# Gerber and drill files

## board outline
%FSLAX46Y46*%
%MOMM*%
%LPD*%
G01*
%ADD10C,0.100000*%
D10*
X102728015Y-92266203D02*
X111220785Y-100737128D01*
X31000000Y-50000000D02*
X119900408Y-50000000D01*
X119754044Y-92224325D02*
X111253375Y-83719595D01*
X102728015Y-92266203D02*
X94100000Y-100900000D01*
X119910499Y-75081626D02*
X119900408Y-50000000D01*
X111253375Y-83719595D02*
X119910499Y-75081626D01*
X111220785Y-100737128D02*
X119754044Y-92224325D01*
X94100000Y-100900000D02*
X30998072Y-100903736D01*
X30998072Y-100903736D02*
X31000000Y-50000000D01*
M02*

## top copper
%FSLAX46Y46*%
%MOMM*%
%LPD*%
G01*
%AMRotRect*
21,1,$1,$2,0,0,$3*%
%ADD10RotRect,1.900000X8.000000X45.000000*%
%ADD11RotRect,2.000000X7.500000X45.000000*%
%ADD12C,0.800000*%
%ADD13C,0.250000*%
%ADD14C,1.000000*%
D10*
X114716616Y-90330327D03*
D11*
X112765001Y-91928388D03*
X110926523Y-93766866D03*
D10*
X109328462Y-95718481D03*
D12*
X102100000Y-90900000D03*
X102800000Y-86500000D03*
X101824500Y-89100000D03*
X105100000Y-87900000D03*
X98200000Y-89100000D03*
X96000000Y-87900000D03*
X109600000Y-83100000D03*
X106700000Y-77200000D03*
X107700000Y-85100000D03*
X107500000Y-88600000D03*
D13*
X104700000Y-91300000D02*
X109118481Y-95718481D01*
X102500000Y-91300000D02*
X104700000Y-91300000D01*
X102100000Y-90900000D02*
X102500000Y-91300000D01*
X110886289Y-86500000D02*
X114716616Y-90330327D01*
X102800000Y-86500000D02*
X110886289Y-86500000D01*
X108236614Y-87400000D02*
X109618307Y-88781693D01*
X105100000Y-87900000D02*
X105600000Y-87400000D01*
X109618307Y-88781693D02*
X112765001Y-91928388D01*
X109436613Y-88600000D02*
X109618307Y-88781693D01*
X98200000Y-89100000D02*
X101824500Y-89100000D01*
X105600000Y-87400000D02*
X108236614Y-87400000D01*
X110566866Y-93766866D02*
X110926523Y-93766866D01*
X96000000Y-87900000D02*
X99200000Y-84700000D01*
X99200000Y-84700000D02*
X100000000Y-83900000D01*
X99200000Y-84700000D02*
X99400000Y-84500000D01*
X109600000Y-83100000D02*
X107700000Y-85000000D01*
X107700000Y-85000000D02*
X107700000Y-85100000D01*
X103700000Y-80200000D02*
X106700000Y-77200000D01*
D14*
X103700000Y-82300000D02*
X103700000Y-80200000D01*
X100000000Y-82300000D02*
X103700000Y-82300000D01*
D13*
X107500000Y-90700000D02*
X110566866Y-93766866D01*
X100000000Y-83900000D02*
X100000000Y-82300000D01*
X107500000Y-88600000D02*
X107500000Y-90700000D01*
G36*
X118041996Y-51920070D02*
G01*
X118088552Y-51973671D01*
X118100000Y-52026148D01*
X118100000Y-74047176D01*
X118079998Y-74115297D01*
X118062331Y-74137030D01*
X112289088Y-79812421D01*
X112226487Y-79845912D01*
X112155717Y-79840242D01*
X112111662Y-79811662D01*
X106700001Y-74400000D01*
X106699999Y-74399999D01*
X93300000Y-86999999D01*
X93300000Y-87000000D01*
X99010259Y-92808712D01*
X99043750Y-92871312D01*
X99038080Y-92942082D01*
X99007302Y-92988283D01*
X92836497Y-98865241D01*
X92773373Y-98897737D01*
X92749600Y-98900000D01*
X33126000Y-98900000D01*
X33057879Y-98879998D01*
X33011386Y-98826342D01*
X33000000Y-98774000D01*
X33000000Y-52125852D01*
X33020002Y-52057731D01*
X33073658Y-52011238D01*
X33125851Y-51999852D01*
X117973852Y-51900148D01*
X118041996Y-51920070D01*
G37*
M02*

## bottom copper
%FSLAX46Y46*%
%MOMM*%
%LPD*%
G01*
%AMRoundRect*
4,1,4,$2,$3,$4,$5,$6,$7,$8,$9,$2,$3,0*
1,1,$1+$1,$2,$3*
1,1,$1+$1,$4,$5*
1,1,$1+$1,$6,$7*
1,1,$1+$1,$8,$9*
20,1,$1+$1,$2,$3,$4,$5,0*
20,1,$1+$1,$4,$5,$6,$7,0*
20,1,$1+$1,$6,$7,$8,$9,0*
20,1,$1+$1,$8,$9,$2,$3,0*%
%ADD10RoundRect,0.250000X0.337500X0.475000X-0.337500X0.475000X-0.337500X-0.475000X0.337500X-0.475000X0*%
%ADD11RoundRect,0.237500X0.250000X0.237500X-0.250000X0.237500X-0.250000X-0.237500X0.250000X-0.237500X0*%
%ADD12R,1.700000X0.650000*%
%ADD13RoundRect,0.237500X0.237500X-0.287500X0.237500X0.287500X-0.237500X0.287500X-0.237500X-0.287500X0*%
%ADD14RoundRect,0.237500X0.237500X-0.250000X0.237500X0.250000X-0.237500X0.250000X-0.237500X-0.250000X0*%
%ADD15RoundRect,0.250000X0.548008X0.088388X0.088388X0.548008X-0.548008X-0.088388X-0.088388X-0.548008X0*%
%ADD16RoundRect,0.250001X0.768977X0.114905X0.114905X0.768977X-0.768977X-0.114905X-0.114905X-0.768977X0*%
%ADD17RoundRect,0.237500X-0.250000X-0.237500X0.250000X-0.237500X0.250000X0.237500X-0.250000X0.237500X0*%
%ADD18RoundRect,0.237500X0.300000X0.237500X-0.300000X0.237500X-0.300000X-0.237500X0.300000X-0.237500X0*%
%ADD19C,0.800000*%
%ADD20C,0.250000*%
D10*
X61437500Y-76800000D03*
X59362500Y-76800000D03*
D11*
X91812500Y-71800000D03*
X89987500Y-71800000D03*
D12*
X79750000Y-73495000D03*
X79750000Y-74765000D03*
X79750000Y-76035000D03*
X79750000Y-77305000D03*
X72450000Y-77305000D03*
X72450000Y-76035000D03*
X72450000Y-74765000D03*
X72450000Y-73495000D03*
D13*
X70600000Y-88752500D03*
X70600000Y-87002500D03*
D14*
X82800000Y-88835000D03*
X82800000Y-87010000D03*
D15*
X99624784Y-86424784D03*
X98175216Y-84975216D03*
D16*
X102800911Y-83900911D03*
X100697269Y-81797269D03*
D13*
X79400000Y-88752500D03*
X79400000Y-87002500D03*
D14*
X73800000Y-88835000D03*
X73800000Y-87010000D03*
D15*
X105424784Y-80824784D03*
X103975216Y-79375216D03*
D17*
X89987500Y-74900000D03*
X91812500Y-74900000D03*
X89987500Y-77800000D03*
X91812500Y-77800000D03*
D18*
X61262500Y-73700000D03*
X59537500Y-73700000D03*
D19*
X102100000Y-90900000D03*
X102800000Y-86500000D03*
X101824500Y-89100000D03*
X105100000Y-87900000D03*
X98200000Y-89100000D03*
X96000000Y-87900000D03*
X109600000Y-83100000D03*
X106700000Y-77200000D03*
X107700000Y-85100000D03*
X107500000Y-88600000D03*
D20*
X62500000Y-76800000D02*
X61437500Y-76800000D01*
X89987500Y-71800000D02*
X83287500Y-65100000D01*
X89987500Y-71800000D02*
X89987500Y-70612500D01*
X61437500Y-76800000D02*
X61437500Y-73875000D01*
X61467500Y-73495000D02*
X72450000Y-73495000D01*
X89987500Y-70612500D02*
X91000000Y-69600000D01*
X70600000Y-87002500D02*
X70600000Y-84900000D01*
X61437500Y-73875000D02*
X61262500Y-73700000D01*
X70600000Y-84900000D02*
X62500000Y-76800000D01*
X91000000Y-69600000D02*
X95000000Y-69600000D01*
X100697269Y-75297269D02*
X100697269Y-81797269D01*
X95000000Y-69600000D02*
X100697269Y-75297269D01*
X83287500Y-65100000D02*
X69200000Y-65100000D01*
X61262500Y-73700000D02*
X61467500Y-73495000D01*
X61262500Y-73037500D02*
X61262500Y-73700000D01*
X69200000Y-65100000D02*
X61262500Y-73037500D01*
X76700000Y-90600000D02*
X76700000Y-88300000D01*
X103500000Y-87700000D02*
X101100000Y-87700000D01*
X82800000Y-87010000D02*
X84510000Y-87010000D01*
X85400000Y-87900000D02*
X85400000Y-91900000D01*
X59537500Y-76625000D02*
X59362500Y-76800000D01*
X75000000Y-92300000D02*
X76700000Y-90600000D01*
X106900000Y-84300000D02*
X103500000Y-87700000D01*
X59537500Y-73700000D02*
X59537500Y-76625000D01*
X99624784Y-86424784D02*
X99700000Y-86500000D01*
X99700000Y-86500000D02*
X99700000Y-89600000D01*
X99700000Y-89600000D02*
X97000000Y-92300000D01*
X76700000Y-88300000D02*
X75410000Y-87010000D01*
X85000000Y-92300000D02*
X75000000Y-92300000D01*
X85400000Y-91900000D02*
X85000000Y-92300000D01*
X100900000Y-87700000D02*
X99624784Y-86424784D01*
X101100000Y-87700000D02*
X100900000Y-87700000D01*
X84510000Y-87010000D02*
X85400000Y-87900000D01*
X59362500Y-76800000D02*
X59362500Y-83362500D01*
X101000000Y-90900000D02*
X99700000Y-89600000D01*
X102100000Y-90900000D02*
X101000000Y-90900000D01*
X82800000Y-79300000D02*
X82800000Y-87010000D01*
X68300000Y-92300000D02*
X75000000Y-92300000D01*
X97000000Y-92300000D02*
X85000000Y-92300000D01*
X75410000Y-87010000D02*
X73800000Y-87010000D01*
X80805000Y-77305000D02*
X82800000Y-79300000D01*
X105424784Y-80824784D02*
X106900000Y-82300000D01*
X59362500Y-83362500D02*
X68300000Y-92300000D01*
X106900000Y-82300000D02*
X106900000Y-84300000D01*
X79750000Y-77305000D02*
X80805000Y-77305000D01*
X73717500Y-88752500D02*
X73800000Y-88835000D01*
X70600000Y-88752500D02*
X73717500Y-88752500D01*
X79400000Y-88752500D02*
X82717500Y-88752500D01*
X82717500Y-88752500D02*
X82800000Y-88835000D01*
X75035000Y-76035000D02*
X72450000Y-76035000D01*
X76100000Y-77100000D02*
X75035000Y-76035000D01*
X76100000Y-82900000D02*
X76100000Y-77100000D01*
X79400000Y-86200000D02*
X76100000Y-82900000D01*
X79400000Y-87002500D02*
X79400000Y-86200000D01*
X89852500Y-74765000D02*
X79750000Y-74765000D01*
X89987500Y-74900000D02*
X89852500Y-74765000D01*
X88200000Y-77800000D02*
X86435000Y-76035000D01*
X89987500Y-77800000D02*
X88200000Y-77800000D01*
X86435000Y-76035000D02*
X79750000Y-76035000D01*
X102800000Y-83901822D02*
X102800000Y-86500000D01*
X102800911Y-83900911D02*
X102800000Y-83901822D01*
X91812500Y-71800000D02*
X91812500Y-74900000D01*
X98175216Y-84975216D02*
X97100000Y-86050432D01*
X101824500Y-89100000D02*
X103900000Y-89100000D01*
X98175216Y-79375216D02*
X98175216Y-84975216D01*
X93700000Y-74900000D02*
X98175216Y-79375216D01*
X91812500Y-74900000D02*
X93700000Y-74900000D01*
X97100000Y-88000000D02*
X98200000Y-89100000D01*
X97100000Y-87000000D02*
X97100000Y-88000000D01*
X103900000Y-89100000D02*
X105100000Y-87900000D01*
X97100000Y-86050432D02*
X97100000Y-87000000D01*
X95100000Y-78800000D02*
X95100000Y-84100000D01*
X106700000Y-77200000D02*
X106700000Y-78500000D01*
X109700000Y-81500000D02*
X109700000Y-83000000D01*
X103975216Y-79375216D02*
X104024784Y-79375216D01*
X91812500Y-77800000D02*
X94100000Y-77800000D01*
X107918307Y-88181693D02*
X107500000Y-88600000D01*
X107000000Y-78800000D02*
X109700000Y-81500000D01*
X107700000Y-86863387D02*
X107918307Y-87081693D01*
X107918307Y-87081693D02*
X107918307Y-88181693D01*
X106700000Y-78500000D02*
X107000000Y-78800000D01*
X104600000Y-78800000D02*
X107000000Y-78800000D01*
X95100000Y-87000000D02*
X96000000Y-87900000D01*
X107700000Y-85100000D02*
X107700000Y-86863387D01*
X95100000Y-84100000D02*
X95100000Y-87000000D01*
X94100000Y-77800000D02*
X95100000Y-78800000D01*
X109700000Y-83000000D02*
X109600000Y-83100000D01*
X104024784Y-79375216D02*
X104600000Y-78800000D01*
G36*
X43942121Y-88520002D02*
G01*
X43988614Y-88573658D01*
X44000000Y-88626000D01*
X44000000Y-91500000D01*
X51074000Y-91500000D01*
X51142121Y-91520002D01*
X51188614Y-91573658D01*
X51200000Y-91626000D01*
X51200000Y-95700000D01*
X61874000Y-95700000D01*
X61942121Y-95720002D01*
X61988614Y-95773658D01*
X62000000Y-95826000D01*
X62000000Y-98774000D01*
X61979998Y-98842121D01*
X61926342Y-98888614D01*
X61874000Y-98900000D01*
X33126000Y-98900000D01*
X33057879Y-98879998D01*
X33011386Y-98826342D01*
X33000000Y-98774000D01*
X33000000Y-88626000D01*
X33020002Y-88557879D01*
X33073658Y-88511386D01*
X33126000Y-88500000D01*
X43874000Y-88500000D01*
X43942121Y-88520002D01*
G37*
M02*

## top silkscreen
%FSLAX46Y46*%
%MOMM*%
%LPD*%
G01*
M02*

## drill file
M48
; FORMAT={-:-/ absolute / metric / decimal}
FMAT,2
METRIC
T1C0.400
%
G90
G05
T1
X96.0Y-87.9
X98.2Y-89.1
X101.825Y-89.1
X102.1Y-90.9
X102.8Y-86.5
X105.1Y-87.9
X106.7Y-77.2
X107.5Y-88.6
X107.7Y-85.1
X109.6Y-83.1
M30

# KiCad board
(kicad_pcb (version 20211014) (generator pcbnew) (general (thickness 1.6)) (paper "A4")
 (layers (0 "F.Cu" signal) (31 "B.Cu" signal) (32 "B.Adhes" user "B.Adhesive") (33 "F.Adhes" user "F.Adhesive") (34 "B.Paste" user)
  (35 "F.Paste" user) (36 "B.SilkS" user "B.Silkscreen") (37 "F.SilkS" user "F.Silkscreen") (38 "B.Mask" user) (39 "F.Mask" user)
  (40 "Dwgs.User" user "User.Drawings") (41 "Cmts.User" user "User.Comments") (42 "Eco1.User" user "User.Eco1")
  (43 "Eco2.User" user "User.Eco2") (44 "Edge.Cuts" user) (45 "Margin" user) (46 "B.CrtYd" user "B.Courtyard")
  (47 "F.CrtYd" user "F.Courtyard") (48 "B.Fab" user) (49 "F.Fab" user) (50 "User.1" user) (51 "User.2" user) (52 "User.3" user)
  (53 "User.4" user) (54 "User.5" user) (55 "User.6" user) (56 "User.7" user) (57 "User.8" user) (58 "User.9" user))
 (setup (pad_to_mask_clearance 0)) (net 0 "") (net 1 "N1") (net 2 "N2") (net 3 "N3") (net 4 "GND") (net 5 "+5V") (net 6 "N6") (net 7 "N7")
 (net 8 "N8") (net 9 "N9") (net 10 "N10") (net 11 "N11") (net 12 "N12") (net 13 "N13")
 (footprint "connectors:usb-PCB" (layer "F.Cu") (at 115.487362 96.489227 45)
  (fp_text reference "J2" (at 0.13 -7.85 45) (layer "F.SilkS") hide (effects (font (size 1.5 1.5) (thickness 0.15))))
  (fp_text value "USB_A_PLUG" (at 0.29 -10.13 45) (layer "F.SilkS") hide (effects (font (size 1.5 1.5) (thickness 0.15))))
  (pad "1" connect rect (at 3.81 -4.9 45) (size 1.9 8) (layers "F.Cu" "F.Mask") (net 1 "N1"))
  (pad "2" connect rect (at 1.3 -5.15 45) (size 2 7.5) (layers "F.Cu" "F.Mask") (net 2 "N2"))
  (pad "3" connect rect (at -1.3 -5.15 45) (size 2 7.5) (layers "F.Cu" "F.Mask") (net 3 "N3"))
  (pad "4" connect rect (at -3.81 -4.9 45) (size 1.9 8) (layers "F.Cu" "F.Mask") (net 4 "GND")))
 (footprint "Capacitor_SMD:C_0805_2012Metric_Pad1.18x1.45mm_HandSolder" (layer "B.Cu") (at 60.4 76.8 180)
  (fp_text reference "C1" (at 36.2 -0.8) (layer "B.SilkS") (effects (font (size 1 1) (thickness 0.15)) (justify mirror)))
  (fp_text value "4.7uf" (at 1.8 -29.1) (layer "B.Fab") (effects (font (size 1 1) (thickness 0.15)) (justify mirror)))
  (pad "1" smd roundrect (at -1.0375 0 180) (size 1.175 1.45) (layers "B.Cu" "B.Paste" "B.Mask") (roundrect_rratio 0.2127659574)
   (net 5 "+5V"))
  (pad "2" smd roundrect (at 1.0375 0 180) (size 1.175 1.45) (layers "B.Cu" "B.Paste" "B.Mask") (roundrect_rratio 0.2127659574)
   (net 4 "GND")))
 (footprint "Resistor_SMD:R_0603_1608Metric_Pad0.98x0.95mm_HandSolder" (layer "B.Cu") (at 90.9 71.8 180)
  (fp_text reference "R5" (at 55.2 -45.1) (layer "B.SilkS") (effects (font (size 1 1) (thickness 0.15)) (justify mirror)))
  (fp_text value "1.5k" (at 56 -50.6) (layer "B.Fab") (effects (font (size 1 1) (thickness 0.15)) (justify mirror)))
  (pad "1" smd roundrect (at -0.9125 0 180) (size 0.975 0.95) (layers "B.Cu" "B.Paste" "B.Mask") (roundrect_rratio 0.25) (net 2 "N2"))
  (pad "2" smd roundrect (at 0.9125 0 180) (size 0.975 0.95) (layers "B.Cu" "B.Paste" "B.Mask") (roundrect_rratio 0.25) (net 5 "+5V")))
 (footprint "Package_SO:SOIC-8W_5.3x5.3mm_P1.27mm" (layer "B.Cu") (at 76.1 75.4 180)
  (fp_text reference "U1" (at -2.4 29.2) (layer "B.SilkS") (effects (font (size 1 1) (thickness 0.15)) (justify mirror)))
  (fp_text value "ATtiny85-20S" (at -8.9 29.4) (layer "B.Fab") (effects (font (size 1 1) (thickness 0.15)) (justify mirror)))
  (pad "1" smd rect (at -3.65 1.905 180) (size 1.7 0.65) (layers "B.Cu" "B.Paste" "B.Mask") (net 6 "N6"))
  (pad "2" smd rect (at -3.65 0.635 180) (size 1.7 0.65) (layers "B.Cu" "B.Paste" "B.Mask") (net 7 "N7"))
  (pad "3" smd rect (at -3.65 -0.635 180) (size 1.7 0.65) (layers "B.Cu" "B.Paste" "B.Mask") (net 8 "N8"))
  (pad "4" smd rect (at -3.65 -1.905 180) (size 1.7 0.65) (layers "B.Cu" "B.Paste" "B.Mask") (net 4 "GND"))
  (pad "5" smd rect (at 3.65 -1.905 180) (size 1.7 0.65) (layers "B.Cu" "B.Paste" "B.Mask") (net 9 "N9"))
  (pad "6" smd rect (at 3.65 -0.635 180) (size 1.7 0.65) (layers "B.Cu" "B.Paste" "B.Mask") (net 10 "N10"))
  (pad "7" smd rect (at 3.65 0.635 180) (size 1.7 0.65) (layers "B.Cu" "B.Paste" "B.Mask") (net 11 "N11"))
  (pad "8" smd rect (at 3.65 1.905 180) (size 1.7 0.65) (layers "B.Cu" "B.Paste" "B.Mask") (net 5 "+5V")))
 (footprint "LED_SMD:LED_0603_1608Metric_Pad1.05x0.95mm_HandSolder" (layer "B.Cu") (at 70.6 87.8775 90)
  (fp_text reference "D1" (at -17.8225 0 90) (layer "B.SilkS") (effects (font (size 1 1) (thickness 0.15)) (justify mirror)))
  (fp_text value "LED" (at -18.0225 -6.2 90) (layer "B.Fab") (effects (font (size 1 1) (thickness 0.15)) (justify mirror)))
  (pad "1" smd roundrect (at -0.875 0 90) (size 1.05 0.95) (layers "B.Cu" "B.Paste" "B.Mask") (roundrect_rratio 0.25) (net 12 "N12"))
  (pad "2" smd roundrect (at 0.875 0 90) (size 1.05 0.95) (layers "B.Cu" "B.Paste" "B.Mask") (roundrect_rratio 0.25) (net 5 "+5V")))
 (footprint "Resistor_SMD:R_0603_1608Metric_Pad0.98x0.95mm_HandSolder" (layer "B.Cu") (at 82.8 87.9225 90)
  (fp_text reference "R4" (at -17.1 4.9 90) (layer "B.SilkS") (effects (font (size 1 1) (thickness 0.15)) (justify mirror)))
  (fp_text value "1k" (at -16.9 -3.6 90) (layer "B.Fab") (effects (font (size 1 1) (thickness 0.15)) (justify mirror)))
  (pad "1" smd roundrect (at -0.9125 0 90) (size 0.975 0.95) (layers "B.Cu" "B.Paste" "B.Mask") (roundrect_rratio 0.25) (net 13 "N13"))
  (pad "2" smd roundrect (at 0.9125 0 90) (size 0.975 0.95) (layers "B.Cu" "B.Paste" "B.Mask") (roundrect_rratio 0.25) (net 4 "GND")))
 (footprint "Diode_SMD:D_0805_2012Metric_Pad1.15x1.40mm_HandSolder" (layer "B.Cu") (at 98.9 85.7 135)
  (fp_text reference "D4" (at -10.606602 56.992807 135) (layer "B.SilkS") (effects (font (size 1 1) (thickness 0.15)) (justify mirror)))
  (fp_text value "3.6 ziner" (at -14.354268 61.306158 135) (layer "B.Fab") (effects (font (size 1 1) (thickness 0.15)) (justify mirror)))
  (pad "1" smd roundrect (at -1.025 0 135) (size 1.15 1.4) (layers "B.Cu" "B.Paste" "B.Mask") (roundrect_rratio 0.2173913043) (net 4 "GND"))
  (pad "2" smd roundrect (at 1.025 0 135) (size 1.15 1.4) (layers "B.Cu" "B.Paste" "B.Mask") (roundrect_rratio 0.2173913043) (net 2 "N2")))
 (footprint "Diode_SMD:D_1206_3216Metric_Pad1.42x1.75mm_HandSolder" (layer "B.Cu") (at 101.74909 82.84909 135)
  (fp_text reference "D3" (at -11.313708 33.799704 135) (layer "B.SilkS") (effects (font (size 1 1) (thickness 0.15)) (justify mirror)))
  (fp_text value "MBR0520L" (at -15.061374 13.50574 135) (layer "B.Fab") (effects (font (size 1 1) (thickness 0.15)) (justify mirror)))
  (pad "1" smd roundrect (at -1.4875 0 135) (size 1.425 1.75) (layers "B.Cu" "B.Paste" "B.Mask") (roundrect_rratio 0.1754392982)
   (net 1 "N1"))
  (pad "2" smd roundrect (at 1.4875 0 135) (size 1.425 1.75) (layers "B.Cu" "B.Paste" "B.Mask") (roundrect_rratio 0.1754392982)
   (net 5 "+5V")))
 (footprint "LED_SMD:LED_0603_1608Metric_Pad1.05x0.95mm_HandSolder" (layer "B.Cu") (at 79.4 87.8775 90)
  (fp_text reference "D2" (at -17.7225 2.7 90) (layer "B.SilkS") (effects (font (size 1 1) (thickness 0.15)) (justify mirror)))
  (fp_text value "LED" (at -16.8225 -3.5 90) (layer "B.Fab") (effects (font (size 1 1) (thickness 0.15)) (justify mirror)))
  (pad "1" smd roundrect (at -0.875 0 90) (size 1.05 0.95) (layers "B.Cu" "B.Paste" "B.Mask") (roundrect_rratio 0.25) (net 13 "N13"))
  (pad "2" smd roundrect (at 0.875 0 90) (size 1.05 0.95) (layers "B.Cu" "B.Paste" "B.Mask") (roundrect_rratio 0.25) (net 10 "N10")))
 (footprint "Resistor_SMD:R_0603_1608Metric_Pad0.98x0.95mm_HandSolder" (layer "B.Cu") (at 73.8 87.9225 90)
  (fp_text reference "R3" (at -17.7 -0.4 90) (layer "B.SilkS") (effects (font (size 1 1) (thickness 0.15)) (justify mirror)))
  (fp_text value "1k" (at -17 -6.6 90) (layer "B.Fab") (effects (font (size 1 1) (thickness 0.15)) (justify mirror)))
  (pad "1" smd roundrect (at -0.9125 0 90) (size 0.975 0.95) (layers "B.Cu" "B.Paste" "B.Mask") (roundrect_rratio 0.25) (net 12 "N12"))
  (pad "2" smd roundrect (at 0.9125 0 90) (size 0.975 0.95) (layers "B.Cu" "B.Paste" "B.Mask") (roundrect_rratio 0.25) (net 4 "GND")))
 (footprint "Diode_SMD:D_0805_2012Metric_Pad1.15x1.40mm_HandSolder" (layer "B.Cu") (at 104.7 80.1 135)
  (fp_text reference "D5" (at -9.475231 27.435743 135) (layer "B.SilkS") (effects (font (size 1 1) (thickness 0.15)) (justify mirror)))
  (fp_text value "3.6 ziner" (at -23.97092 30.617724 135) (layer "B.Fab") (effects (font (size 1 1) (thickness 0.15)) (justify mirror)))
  (pad "1" smd roundrect (at -1.025 0 135) (size 1.15 1.4) (layers "B.Cu" "B.Paste" "B.Mask") (roundrect_rratio 0.2173913043) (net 4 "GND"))
  (pad "2" smd roundrect (at 1.025 0 135) (size 1.15 1.4) (layers "B.Cu" "B.Paste" "B.Mask") (roundrect_rratio 0.2173913043) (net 3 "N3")))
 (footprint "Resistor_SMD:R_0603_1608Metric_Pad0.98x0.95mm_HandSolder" (layer "B.Cu") (at 90.9 74.9)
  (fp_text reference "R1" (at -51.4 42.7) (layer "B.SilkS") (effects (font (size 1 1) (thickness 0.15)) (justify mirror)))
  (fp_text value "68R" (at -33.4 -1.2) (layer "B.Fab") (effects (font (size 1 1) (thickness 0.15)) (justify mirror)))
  (pad "1" smd roundrect (at -0.9125 0) (size 0.975 0.95) (layers "B.Cu" "B.Paste" "B.Mask") (roundrect_rratio 0.25) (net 7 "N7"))
  (pad "2" smd roundrect (at 0.9125 0) (size 0.975 0.95) (layers "B.Cu" "B.Paste" "B.Mask") (roundrect_rratio 0.25) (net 2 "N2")))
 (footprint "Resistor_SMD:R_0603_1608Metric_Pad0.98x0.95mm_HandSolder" (layer "B.Cu") (at 90.9 77.8)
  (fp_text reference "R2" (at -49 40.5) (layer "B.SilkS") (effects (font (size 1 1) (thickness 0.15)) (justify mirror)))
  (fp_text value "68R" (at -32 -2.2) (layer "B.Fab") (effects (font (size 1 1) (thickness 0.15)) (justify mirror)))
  (pad "1" smd roundrect (at -0.9125 0) (size 0.975 0.95) (layers "B.Cu" "B.Paste" "B.Mask") (roundrect_rratio 0.25) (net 8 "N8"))
  (pad "2" smd roundrect (at 0.9125 0) (size 0.975 0.95) (layers "B.Cu" "B.Paste" "B.Mask") (roundrect_rratio 0.25) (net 3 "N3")))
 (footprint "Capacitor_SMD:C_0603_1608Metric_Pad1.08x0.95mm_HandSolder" (layer "B.Cu") (at 60.4 73.7 180)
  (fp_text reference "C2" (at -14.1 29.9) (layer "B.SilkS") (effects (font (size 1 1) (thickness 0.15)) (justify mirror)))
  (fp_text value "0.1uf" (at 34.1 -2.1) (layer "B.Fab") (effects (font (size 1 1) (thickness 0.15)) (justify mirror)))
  (pad "1" smd roundrect (at -0.8625 0 180) (size 1.075 0.95) (layers "B.Cu" "B.Paste" "B.Mask") (roundrect_rratio 0.25) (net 5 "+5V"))
  (pad "2" smd roundrect (at 0.8625 0 180) (size 1.075 0.95) (layers "B.Cu" "B.Paste" "B.Mask") (roundrect_rratio 0.25) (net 4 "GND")))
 (gr_line (start 102.728015 92.266203) (end 111.220785 100.737128) (layer "Edge.Cuts") (width 0.1))
 (gr_line (start 31 50) (end 119.900408 50) (layer "Edge.Cuts") (width 0.1))
 (gr_line (start 119.754044 92.224325) (end 111.253375 83.719595) (layer "Edge.Cuts") (width 0.1))
 (gr_line (start 102.728015 92.266203) (end 94.1 100.9) (layer "Edge.Cuts") (width 0.1))
 (gr_line (start 119.910499 75.081626) (end 119.900408 50) (layer "Edge.Cuts") (width 0.1))
 (gr_line (start 111.253375 83.719595) (end 119.910499 75.081626) (layer "Edge.Cuts") (width 0.1))
 (gr_line (start 111.220785 100.737128) (end 119.754044 92.224325) (layer "Edge.Cuts") (width 0.1))
 (gr_line (start 94.1 100.9) (end 30.998072 100.903736) (layer "Edge.Cuts") (width 0.1))
 (gr_line (start 30.998072 100.903736) (end 31 50) (layer "Edge.Cuts") (width 0.1))
 (segment (start 62.5 76.8) (end 61.4375 76.8) (width 0.25) (layer "B.Cu") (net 5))
 (segment (start 89.9875 71.8) (end 83.2875 65.1) (width 0.25) (layer "B.Cu") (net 5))
 (segment (start 89.9875 71.8) (end 89.9875 70.6125) (width 0.25) (layer "B.Cu") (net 5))
 (segment (start 61.4375 76.8) (end 61.4375 73.875) (width 0.25) (layer "B.Cu") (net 5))
 (segment (start 61.4675 73.495) (end 72.45 73.495) (width 0.25) (layer "B.Cu") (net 5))
 (segment (start 89.9875 70.6125) (end 91 69.6) (width 0.25) (layer "B.Cu") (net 5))
 (segment (start 70.6 87.0025) (end 70.6 84.9) (width 0.25) (layer "B.Cu") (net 5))
 (segment (start 61.4375 73.875) (end 61.2625 73.7) (width 0.25) (layer "B.Cu") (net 5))
 (segment (start 70.6 84.9) (end 62.5 76.8) (width 0.25) (layer "B.Cu") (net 5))
 (segment (start 91 69.6) (end 95 69.6) (width 0.25) (layer "B.Cu") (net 5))
 (segment (start 100.697269 75.297269) (end 100.697269 81.797269) (width 0.25) (layer "B.Cu") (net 5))
 (segment (start 95 69.6) (end 100.697269 75.297269) (width 0.25) (layer "B.Cu") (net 5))
 (segment (start 83.2875 65.1) (end 69.2 65.1) (width 0.25) (layer "B.Cu") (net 5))
 (segment (start 61.2625 73.7) (end 61.4675 73.495) (width 0.25) (layer "B.Cu") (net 5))
 (segment (start 61.2625 73.0375) (end 61.2625 73.7) (width 0.25) (layer "B.Cu") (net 5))
 (segment (start 69.2 65.1) (end 61.2625 73.0375) (width 0.25) (layer "B.Cu") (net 5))
 (segment (start 104.7 91.3) (end 109.118481 95.718481) (width 0.25) (layer "F.Cu") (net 4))
 (segment (start 102.5 91.3) (end 104.7 91.3) (width 0.25) (layer "F.Cu") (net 4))
 (segment (start 102.1 90.9) (end 102.5 91.3) (width 0.25) (layer "F.Cu") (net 4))
 (via (at 102.1 90.9) (size 0.8) (drill 0.4) (layers "F.Cu" "B.Cu") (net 4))
 (segment (start 76.7 90.6) (end 76.7 88.3) (width 0.25) (layer "B.Cu") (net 4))
 (segment (start 103.5 87.7) (end 101.1 87.7) (width 0.25) (layer "B.Cu") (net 4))
 (segment (start 82.8 87.01) (end 84.51 87.01) (width 0.25) (layer "B.Cu") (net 4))
 (segment (start 85.4 87.9) (end 85.4 91.9) (width 0.25) (layer "B.Cu") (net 4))
 (segment (start 59.5375 76.625) (end 59.3625 76.8) (width 0.25) (layer "B.Cu") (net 4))
 (segment (start 75 92.3) (end 76.7 90.6) (width 0.25) (layer "B.Cu") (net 4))
 (segment (start 106.9 84.3) (end 103.5 87.7) (width 0.25) (layer "B.Cu") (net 4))
 (segment (start 59.5375 73.7) (end 59.5375 76.625) (width 0.25) (layer "B.Cu") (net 4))
 (segment (start 99.624784 86.424784) (end 99.7 86.5) (width 0.25) (layer "B.Cu") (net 4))
 (segment (start 99.7 86.5) (end 99.7 89.6) (width 0.25) (layer "B.Cu") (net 4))
 (segment (start 99.7 89.6) (end 97 92.3) (width 0.25) (layer "B.Cu") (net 4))
 (segment (start 76.7 88.3) (end 75.41 87.01) (width 0.25) (layer "B.Cu") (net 4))
 (segment (start 85 92.3) (end 75 92.3) (width 0.25) (layer "B.Cu") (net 4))
 (segment (start 85.4 91.9) (end 85 92.3) (width 0.25) (layer "B.Cu") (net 4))
 (segment (start 100.9 87.7) (end 99.624784 86.424784) (width 0.25) (layer "B.Cu") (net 4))
 (segment (start 101.1 87.7) (end 100.9 87.7) (width 0.25) (layer "B.Cu") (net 4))
 (segment (start 84.51 87.01) (end 85.4 87.9) (width 0.25) (layer "B.Cu") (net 4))
 (segment (start 59.3625 76.8) (end 59.3625 83.3625) (width 0.25) (layer "B.Cu") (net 4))
 (segment (start 101 90.9) (end 99.7 89.6) (width 0.25) (layer "B.Cu") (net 4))
 (segment (start 102.1 90.9) (end 101 90.9) (width 0.25) (layer "B.Cu") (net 4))
 (segment (start 82.8 79.3) (end 82.8 87.01) (width 0.25) (layer "B.Cu") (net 4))
 (segment (start 68.3 92.3) (end 75 92.3) (width 0.25) (layer "B.Cu") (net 4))
 (segment (start 97 92.3) (end 85 92.3) (width 0.25) (layer "B.Cu") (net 4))
 (segment (start 75.41 87.01) (end 73.8 87.01) (width 0.25) (layer "B.Cu") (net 4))
 (segment (start 80.805 77.305) (end 82.8 79.3) (width 0.25) (layer "B.Cu") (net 4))
 (segment (start 105.424784 80.824784) (end 106.9 82.3) (width 0.25) (layer "B.Cu") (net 4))
 (segment (start 59.3625 83.3625) (end 68.3 92.3) (width 0.25) (layer "B.Cu") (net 4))
 (segment (start 106.9 82.3) (end 106.9 84.3) (width 0.25) (layer "B.Cu") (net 4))
 (segment (start 79.75 77.305) (end 80.805 77.305) (width 0.25) (layer "B.Cu") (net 4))
 (segment (start 73.7175 88.7525) (end 73.8 88.835) (width 0.25) (layer "B.Cu") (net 12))
 (segment (start 70.6 88.7525) (end 73.7175 88.7525) (width 0.25) (layer "B.Cu") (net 12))
 (segment (start 79.4 88.7525) (end 82.7175 88.7525) (width 0.25) (layer "B.Cu") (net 13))
 (segment (start 82.7175 88.7525) (end 82.8 88.835) (width 0.25) (layer "B.Cu") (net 13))
 (segment (start 75.035 76.035) (end 72.45 76.035) (width 0.25) (layer "B.Cu") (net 10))
 (segment (start 76.1 77.1) (end 75.035 76.035) (width 0.25) (layer "B.Cu") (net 10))
 (segment (start 76.1 82.9) (end 76.1 77.1) (width 0.25) (layer "B.Cu") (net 10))
 (segment (start 79.4 86.2) (end 76.1 82.9) (width 0.25) (layer "B.Cu") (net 10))
 (segment (start 79.4 87.0025) (end 79.4 86.2) (width 0.25) (layer "B.Cu") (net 10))
 (segment (start 89.8525 74.765) (end 79.75 74.765) (width 0.25) (layer "B.Cu") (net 7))
 (segment (start 89.9875 74.9) (end 89.8525 74.765) (width 0.25) (layer "B.Cu") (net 7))
 (segment (start 88.2 77.8) (end 86.435 76.035) (width 0.25) (layer "B.Cu") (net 8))
 (segment (start 89.9875 77.8) (end 88.2 77.8) (width 0.25) (layer "B.Cu") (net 8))
 (segment (start 86.435 76.035) (end 79.75 76.035) (width 0.25) (layer "B.Cu") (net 8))
 (segment (start 110.886289 86.5) (end 114.716616 90.330327) (width 0.25) (layer "F.Cu") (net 1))
 (segment (start 102.8 86.5) (end 110.886289 86.5) (width 0.25) (layer "F.Cu") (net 1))
 (via (at 102.8 86.5) (size 0.8) (drill 0.4) (layers "F.Cu" "B.Cu") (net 1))
 (segment (start 102.8 83.901822) (end 102.8 86.5) (width 0.25) (layer "B.Cu") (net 1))
 (segment (start 102.800911 83.900911) (end 102.8 83.901822) (width 0.25) (layer "B.Cu") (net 1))
 (segment (start 108.236614 87.4) (end 109.618307 88.781693) (width 0.25) (layer "F.Cu") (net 2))
 (segment (start 105.1 87.9) (end 105.6 87.4) (width 0.25) (layer "F.Cu") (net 2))
 (segment (start 109.618307 88.781693) (end 112.765001 91.928388) (width 0.25) (layer "F.Cu") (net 2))
 (segment (start 109.436613 88.6) (end 109.618307 88.781693) (width 0.25) (layer "F.Cu") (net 2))
 (segment (start 98.2 89.1) (end 101.8245 89.1) (width 0.25) (layer "F.Cu") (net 2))
 (segment (start 105.6 87.4) (end 108.236614 87.4) (width 0.25) (layer "F.Cu") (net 2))
 (via (at 101.8245 89.1) (size 0.8) (drill 0.4) (layers "F.Cu" "B.Cu") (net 2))
 (via (at 105.1 87.9) (size 0.8) (drill 0.4) (layers "F.Cu" "B.Cu") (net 2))
 (via (at 98.2 89.1) (size 0.8) (drill 0.4) (layers "F.Cu" "B.Cu") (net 2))
 (segment (start 91.8125 71.8) (end 91.8125 74.9) (width 0.25) (layer "B.Cu") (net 2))
 (segment (start 98.175216 84.975216) (end 97.1 86.050432) (width 0.25) (layer "B.Cu") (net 2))
 (segment (start 101.8245 89.1) (end 103.9 89.1) (width 0.25) (layer "B.Cu") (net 2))
 (segment (start 98.175216 79.375216) (end 98.175216 84.975216) (width 0.25) (layer "B.Cu") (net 2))
 (segment (start 93.7 74.9) (end 98.175216 79.375216) (width 0.25) (layer "B.Cu") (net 2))
 (segment (start 91.8125 74.9) (end 93.7 74.9) (width 0.25) (layer "B.Cu") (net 2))
 (segment (start 97.1 88) (end 98.2 89.1) (width 0.25) (layer "B.Cu") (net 2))
 (segment (start 97.1 87) (end 97.1 88) (width 0.25) (layer "B.Cu") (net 2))
 (segment (start 103.9 89.1) (end 105.1 87.9) (width 0.25) (layer "B.Cu") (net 2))
 (segment (start 97.1 86.050432) (end 97.1 87) (width 0.25) (layer "B.Cu") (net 2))
 (segment (start 110.566866 93.766866) (end 110.926523 93.766866) (width 0.25) (layer "F.Cu") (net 3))
 (segment (start 96 87.9) (end 99.2 84.7) (width 0.25) (layer "F.Cu") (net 3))
 (segment (start 99.2 84.7) (end 100 83.9) (width 0.25) (layer "F.Cu") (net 3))
 (segment (start 99.2 84.7) (end 99.4 84.5) (width 0.25) (layer "F.Cu") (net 3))
 (segment (start 109.6 83.1) (end 107.7 85) (width 0.25) (layer "F.Cu") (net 3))
 (segment (start 107.7 85) (end 107.7 85.1) (width 0.25) (layer "F.Cu") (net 3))
 (segment (start 103.7 80.2) (end 106.7 77.2) (width 0.25) (layer "F.Cu") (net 3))
 (segment (start 103.7 82.3) (end 103.7 80.2) (width 1) (layer "F.Cu") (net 3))
 (segment (start 100 82.3) (end 103.7 82.3) (width 1) (layer "F.Cu") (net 3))
 (segment (start 107.5 90.7) (end 110.566866 93.766866) (width 0.25) (layer "F.Cu") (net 3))
 (segment (start 100 83.9) (end 100 82.3) (width 0.25) (layer "F.Cu") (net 3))
 (segment (start 107.5 88.6) (end 107.5 90.7) (width 0.25) (layer "F.Cu") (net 3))
 (via (at 96 87.9) (size 0.8) (drill 0.4) (layers "F.Cu" "B.Cu") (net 3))
 (via (at 109.6 83.1) (size 0.8) (drill 0.4) (layers "F.Cu" "B.Cu") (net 3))
 (via (at 106.7 77.2) (size 0.8) (drill 0.4) (layers "F.Cu" "B.Cu") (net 3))
 (via (at 107.7 85.1) (size 0.8) (drill 0.4) (layers "F.Cu" "B.Cu") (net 3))
 (via (at 107.5 88.6) (size 0.8) (drill 0.4) (layers "F.Cu" "B.Cu") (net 3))
 (segment (start 95.1 78.8) (end 95.1 84.1) (width 0.25) (layer "B.Cu") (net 3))
 (segment (start 106.7 77.2) (end 106.7 78.5) (width 0.25) (layer "B.Cu") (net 3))
 (segment (start 109.7 81.5) (end 109.7 83) (width 0.25) (layer "B.Cu") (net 3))
 (segment (start 103.975216 79.375216) (end 104.024784 79.375216) (width 0.25) (layer "B.Cu") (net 3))
 (segment (start 91.8125 77.8) (end 94.1 77.8) (width 0.25) (layer "B.Cu") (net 3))
 (segment (start 107.918307 88.181693) (end 107.5 88.6) (width 0.25) (layer "B.Cu") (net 3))
 (segment (start 107 78.8) (end 109.7 81.5) (width 0.25) (layer "B.Cu") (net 3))
 (segment (start 107.7 86.863387) (end 107.918307 87.081693) (width 0.25) (layer "B.Cu") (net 3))
 (segment (start 107.918307 87.081693) (end 107.918307 88.181693) (width 0.25) (layer "B.Cu") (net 3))
 (segment (start 106.7 78.5) (end 107 78.8) (width 0.25) (layer "B.Cu") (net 3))
 (segment (start 104.6 78.8) (end 107 78.8) (width 0.25) (layer "B.Cu") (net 3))
 (segment (start 95.1 87) (end 96 87.9) (width 0.25) (layer "B.Cu") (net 3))
 (segment (start 107.7 85.1) (end 107.7 86.863387) (width 0.25) (layer "B.Cu") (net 3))
 (segment (start 95.1 84.1) (end 95.1 87) (width 0.25) (layer "B.Cu") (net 3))
 (segment (start 94.1 77.8) (end 95.1 78.8) (width 0.25) (layer "B.Cu") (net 3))
 (segment (start 109.7 83) (end 109.6 83.1) (width 0.25) (layer "B.Cu") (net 3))
 (segment (start 104.024784 79.375216) (end 104.6 78.8) (width 0.25) (layer "B.Cu") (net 3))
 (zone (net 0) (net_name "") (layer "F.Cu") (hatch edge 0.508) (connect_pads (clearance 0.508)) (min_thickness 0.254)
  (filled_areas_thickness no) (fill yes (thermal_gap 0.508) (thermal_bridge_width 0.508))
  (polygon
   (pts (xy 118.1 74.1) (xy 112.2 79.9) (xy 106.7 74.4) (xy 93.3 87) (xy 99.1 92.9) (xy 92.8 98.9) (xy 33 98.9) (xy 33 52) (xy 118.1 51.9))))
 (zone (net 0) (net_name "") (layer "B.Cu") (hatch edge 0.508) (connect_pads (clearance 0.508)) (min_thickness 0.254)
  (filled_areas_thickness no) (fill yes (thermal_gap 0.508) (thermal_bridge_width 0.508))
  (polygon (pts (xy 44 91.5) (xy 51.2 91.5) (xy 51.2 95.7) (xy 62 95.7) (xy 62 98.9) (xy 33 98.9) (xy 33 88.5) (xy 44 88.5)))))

